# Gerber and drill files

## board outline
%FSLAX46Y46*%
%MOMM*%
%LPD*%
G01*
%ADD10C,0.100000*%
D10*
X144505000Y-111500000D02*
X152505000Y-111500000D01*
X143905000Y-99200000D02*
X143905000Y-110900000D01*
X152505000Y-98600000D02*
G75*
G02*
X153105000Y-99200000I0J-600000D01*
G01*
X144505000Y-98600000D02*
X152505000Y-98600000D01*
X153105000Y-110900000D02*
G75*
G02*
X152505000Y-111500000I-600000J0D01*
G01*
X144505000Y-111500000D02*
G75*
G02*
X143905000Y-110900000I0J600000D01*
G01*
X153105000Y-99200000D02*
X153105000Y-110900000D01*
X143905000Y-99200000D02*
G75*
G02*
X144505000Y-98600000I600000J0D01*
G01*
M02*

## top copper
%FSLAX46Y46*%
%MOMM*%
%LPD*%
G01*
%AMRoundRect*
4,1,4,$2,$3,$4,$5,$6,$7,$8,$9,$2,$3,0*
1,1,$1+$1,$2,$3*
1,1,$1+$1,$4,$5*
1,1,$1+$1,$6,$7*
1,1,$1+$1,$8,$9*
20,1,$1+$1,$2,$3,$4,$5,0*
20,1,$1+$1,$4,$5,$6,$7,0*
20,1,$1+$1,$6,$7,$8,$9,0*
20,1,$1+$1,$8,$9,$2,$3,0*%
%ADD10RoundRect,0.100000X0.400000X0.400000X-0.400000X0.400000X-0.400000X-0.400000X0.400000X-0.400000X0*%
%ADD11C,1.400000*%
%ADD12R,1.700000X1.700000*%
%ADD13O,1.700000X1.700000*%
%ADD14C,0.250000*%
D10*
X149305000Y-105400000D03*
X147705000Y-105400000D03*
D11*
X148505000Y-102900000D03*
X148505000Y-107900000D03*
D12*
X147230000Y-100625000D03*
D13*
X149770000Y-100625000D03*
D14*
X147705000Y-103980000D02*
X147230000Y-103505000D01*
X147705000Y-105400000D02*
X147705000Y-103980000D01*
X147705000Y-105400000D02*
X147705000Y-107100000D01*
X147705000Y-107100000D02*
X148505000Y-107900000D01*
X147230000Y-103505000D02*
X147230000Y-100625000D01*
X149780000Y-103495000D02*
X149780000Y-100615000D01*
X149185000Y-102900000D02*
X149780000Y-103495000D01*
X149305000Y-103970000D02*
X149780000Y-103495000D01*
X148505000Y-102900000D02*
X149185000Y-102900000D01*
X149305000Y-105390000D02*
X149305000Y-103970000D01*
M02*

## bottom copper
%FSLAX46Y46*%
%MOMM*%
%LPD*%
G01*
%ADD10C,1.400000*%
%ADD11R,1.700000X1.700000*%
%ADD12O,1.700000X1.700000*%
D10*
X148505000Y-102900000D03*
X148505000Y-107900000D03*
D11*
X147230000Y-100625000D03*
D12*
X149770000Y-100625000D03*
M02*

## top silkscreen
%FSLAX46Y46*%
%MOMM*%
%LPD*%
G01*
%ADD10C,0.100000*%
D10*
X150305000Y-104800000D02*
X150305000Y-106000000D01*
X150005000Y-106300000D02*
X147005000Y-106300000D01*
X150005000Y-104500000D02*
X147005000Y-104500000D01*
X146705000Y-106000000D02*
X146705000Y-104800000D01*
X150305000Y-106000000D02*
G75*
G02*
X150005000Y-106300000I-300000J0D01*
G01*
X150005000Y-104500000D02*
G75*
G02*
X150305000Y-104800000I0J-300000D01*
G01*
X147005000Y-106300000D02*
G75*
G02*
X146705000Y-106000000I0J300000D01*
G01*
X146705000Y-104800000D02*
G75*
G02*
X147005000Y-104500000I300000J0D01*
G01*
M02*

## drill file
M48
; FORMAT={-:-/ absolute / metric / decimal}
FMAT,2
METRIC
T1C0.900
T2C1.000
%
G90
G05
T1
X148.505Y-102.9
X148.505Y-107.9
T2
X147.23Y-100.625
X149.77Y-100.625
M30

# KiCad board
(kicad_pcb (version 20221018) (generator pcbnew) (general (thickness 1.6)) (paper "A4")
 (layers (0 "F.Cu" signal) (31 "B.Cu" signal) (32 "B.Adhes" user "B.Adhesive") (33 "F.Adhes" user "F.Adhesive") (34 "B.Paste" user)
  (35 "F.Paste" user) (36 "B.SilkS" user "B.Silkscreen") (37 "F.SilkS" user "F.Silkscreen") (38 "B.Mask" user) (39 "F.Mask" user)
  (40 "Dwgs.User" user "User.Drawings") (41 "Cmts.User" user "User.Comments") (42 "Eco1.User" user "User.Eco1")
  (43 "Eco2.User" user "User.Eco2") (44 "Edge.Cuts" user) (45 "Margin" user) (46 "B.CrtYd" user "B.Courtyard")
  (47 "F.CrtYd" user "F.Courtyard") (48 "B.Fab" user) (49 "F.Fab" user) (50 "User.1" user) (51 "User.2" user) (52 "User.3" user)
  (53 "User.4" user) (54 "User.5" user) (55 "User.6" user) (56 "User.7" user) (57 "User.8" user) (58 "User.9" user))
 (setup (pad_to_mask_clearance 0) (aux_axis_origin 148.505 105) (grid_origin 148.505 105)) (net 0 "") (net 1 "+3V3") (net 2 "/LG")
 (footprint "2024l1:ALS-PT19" (layer "F.Cu") (at 148.505 105.4 180)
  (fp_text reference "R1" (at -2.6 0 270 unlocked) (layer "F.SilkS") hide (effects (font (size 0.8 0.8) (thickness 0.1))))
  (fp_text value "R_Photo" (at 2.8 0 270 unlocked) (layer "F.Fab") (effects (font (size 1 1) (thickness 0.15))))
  (fp_line (start -1.8 0.6) (end -1.8 -0.6) (stroke (width 0.1) (type default)) (layer "F.SilkS"))
  (fp_line (start -1.5 -0.9) (end 1.5 -0.9) (stroke (width 0.1) (type default)) (layer "F.SilkS"))
  (fp_line (start -1.5 0.9) (end 1.5 0.9) (stroke (width 0.1) (type default)) (layer "F.SilkS"))
  (fp_line (start 1.8 -0.6) (end 1.8 0.6) (stroke (width 0.1) (type default)) (layer "F.SilkS"))
  (fp_arc (start -1.8 -0.6) (mid -1.712132 -0.812132) (end -1.5 -0.9) (stroke (width 0.1) (type default)) (layer "F.SilkS"))
  (fp_arc (start -1.5 0.9) (mid -1.712132 0.812132) (end -1.8 0.6) (stroke (width 0.1) (type default)) (layer "F.SilkS"))
  (fp_arc (start 1.5 -0.9) (mid 1.712132 -0.812132) (end 1.8 -0.6) (stroke (width 0.1) (type default)) (layer "F.SilkS"))
  (fp_arc (start 1.8 0.6) (mid 1.712132 0.812132) (end 1.5 0.9) (stroke (width 0.1) (type default)) (layer "F.SilkS"))
  (pad "1" smd roundrect (at -0.8 0 180) (size 1 1) (layers "F.Cu" "F.Mask") (roundrect_rratio 0.1) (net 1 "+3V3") (solder_mask_margin 0.1)
   (thermal_bridge_angle 45))
  (pad "2" smd roundrect (at 0.8 0 180) (size 1 1) (layers "F.Cu" "F.Mask") (roundrect_rratio 0.1) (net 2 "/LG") (solder_mask_margin 0.1)
   (thermal_bridge_angle 45)))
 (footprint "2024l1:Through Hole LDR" (layer "F.Cu") (at 148.505 105.4 90)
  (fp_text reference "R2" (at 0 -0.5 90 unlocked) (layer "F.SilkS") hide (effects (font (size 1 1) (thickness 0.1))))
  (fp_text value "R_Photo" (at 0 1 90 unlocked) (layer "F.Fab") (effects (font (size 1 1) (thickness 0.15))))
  (pad "1" thru_hole circle (at 2.5 0 90) (size 1.4 1.4) (drill 0.9) (layers "*.Cu" "*.Mask") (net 1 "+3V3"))
  (pad "2" thru_hole circle (at -2.5 0 90) (size 1.4 1.4) (drill 0.9) (layers "*.Cu" "*.Mask") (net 2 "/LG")))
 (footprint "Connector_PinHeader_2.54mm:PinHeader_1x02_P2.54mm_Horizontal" (layer "B.Cu") (at 147.23 100.625 -90)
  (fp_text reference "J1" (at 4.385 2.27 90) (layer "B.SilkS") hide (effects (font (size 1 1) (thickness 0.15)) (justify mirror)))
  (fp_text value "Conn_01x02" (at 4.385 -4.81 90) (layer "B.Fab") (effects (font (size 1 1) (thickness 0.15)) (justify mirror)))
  (pad "1" thru_hole rect (at 0 0 270) (size 1.7 1.7) (drill 1) (layers "*.Cu" "*.Mask") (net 2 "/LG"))
  (pad "2" thru_hole oval (at 0 -2.54 270) (size 1.7 1.7) (drill 1) (layers "*.Cu" "*.Mask") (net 1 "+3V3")))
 (gr_line (start 144.505 111.5) (end 152.505 111.5) (stroke (width 0.1) (type default)) (layer "Edge.Cuts"))
 (gr_line (start 143.905 99.2) (end 143.905 110.9) (stroke (width 0.1) (type default)) (layer "Edge.Cuts"))
 (gr_arc (start 152.505 98.6) (mid 152.929264 98.775736) (end 153.105 99.2) (stroke (width 0.1) (type default)) (layer "Edge.Cuts"))
 (gr_line (start 144.505 98.6) (end 152.505 98.6) (stroke (width 0.1) (type default)) (layer "Edge.Cuts"))
 (gr_arc (start 153.105 110.9) (mid 152.929264 111.324264) (end 152.505 111.5) (stroke (width 0.1) (type default)) (layer "Edge.Cuts"))
 (gr_arc (start 144.505 111.5) (mid 144.080736 111.324264) (end 143.905 110.9) (stroke (width 0.1) (type default)) (layer "Edge.Cuts"))
 (gr_line (start 153.105 99.2) (end 153.105 110.9) (stroke (width 0.1) (type default)) (layer "Edge.Cuts"))
 (gr_arc (start 143.905 99.2) (mid 144.080736 98.775736) (end 144.505 98.6) (stroke (width 0.1) (type default)) (layer "Edge.Cuts"))
 (segment (start 147.705 103.98) (end 147.23 103.505) (width 0.25) (layer "F.Cu") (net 2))
 (segment (start 147.705 105.4) (end 147.705 103.98) (width 0.25) (layer "F.Cu") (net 2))
 (segment (start 147.705 105.4) (end 147.705 107.1) (width 0.25) (layer "F.Cu") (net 2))
 (segment (start 147.705 107.1) (end 148.505 107.9) (width 0.25) (layer "F.Cu") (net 2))
 (segment (start 147.23 103.505) (end 147.23 100.625) (width 0.25) (layer "F.Cu") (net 2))
 (segment (start 149.78 103.495) (end 149.78 100.615) (width 0.25) (layer "F.Cu") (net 1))
 (segment (start 149.185 102.9) (end 149.78 103.495) (width 0.25) (layer "F.Cu") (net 1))
 (segment (start 149.305 103.97) (end 149.78 103.495) (width 0.25) (layer "F.Cu") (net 1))
 (segment (start 148.505 102.9) (end 149.185 102.9) (width 0.25) (layer "F.Cu") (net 1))
 (segment (start 149.305 105.39) (end 149.305 103.97) (width 0.25) (layer "F.Cu") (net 1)))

